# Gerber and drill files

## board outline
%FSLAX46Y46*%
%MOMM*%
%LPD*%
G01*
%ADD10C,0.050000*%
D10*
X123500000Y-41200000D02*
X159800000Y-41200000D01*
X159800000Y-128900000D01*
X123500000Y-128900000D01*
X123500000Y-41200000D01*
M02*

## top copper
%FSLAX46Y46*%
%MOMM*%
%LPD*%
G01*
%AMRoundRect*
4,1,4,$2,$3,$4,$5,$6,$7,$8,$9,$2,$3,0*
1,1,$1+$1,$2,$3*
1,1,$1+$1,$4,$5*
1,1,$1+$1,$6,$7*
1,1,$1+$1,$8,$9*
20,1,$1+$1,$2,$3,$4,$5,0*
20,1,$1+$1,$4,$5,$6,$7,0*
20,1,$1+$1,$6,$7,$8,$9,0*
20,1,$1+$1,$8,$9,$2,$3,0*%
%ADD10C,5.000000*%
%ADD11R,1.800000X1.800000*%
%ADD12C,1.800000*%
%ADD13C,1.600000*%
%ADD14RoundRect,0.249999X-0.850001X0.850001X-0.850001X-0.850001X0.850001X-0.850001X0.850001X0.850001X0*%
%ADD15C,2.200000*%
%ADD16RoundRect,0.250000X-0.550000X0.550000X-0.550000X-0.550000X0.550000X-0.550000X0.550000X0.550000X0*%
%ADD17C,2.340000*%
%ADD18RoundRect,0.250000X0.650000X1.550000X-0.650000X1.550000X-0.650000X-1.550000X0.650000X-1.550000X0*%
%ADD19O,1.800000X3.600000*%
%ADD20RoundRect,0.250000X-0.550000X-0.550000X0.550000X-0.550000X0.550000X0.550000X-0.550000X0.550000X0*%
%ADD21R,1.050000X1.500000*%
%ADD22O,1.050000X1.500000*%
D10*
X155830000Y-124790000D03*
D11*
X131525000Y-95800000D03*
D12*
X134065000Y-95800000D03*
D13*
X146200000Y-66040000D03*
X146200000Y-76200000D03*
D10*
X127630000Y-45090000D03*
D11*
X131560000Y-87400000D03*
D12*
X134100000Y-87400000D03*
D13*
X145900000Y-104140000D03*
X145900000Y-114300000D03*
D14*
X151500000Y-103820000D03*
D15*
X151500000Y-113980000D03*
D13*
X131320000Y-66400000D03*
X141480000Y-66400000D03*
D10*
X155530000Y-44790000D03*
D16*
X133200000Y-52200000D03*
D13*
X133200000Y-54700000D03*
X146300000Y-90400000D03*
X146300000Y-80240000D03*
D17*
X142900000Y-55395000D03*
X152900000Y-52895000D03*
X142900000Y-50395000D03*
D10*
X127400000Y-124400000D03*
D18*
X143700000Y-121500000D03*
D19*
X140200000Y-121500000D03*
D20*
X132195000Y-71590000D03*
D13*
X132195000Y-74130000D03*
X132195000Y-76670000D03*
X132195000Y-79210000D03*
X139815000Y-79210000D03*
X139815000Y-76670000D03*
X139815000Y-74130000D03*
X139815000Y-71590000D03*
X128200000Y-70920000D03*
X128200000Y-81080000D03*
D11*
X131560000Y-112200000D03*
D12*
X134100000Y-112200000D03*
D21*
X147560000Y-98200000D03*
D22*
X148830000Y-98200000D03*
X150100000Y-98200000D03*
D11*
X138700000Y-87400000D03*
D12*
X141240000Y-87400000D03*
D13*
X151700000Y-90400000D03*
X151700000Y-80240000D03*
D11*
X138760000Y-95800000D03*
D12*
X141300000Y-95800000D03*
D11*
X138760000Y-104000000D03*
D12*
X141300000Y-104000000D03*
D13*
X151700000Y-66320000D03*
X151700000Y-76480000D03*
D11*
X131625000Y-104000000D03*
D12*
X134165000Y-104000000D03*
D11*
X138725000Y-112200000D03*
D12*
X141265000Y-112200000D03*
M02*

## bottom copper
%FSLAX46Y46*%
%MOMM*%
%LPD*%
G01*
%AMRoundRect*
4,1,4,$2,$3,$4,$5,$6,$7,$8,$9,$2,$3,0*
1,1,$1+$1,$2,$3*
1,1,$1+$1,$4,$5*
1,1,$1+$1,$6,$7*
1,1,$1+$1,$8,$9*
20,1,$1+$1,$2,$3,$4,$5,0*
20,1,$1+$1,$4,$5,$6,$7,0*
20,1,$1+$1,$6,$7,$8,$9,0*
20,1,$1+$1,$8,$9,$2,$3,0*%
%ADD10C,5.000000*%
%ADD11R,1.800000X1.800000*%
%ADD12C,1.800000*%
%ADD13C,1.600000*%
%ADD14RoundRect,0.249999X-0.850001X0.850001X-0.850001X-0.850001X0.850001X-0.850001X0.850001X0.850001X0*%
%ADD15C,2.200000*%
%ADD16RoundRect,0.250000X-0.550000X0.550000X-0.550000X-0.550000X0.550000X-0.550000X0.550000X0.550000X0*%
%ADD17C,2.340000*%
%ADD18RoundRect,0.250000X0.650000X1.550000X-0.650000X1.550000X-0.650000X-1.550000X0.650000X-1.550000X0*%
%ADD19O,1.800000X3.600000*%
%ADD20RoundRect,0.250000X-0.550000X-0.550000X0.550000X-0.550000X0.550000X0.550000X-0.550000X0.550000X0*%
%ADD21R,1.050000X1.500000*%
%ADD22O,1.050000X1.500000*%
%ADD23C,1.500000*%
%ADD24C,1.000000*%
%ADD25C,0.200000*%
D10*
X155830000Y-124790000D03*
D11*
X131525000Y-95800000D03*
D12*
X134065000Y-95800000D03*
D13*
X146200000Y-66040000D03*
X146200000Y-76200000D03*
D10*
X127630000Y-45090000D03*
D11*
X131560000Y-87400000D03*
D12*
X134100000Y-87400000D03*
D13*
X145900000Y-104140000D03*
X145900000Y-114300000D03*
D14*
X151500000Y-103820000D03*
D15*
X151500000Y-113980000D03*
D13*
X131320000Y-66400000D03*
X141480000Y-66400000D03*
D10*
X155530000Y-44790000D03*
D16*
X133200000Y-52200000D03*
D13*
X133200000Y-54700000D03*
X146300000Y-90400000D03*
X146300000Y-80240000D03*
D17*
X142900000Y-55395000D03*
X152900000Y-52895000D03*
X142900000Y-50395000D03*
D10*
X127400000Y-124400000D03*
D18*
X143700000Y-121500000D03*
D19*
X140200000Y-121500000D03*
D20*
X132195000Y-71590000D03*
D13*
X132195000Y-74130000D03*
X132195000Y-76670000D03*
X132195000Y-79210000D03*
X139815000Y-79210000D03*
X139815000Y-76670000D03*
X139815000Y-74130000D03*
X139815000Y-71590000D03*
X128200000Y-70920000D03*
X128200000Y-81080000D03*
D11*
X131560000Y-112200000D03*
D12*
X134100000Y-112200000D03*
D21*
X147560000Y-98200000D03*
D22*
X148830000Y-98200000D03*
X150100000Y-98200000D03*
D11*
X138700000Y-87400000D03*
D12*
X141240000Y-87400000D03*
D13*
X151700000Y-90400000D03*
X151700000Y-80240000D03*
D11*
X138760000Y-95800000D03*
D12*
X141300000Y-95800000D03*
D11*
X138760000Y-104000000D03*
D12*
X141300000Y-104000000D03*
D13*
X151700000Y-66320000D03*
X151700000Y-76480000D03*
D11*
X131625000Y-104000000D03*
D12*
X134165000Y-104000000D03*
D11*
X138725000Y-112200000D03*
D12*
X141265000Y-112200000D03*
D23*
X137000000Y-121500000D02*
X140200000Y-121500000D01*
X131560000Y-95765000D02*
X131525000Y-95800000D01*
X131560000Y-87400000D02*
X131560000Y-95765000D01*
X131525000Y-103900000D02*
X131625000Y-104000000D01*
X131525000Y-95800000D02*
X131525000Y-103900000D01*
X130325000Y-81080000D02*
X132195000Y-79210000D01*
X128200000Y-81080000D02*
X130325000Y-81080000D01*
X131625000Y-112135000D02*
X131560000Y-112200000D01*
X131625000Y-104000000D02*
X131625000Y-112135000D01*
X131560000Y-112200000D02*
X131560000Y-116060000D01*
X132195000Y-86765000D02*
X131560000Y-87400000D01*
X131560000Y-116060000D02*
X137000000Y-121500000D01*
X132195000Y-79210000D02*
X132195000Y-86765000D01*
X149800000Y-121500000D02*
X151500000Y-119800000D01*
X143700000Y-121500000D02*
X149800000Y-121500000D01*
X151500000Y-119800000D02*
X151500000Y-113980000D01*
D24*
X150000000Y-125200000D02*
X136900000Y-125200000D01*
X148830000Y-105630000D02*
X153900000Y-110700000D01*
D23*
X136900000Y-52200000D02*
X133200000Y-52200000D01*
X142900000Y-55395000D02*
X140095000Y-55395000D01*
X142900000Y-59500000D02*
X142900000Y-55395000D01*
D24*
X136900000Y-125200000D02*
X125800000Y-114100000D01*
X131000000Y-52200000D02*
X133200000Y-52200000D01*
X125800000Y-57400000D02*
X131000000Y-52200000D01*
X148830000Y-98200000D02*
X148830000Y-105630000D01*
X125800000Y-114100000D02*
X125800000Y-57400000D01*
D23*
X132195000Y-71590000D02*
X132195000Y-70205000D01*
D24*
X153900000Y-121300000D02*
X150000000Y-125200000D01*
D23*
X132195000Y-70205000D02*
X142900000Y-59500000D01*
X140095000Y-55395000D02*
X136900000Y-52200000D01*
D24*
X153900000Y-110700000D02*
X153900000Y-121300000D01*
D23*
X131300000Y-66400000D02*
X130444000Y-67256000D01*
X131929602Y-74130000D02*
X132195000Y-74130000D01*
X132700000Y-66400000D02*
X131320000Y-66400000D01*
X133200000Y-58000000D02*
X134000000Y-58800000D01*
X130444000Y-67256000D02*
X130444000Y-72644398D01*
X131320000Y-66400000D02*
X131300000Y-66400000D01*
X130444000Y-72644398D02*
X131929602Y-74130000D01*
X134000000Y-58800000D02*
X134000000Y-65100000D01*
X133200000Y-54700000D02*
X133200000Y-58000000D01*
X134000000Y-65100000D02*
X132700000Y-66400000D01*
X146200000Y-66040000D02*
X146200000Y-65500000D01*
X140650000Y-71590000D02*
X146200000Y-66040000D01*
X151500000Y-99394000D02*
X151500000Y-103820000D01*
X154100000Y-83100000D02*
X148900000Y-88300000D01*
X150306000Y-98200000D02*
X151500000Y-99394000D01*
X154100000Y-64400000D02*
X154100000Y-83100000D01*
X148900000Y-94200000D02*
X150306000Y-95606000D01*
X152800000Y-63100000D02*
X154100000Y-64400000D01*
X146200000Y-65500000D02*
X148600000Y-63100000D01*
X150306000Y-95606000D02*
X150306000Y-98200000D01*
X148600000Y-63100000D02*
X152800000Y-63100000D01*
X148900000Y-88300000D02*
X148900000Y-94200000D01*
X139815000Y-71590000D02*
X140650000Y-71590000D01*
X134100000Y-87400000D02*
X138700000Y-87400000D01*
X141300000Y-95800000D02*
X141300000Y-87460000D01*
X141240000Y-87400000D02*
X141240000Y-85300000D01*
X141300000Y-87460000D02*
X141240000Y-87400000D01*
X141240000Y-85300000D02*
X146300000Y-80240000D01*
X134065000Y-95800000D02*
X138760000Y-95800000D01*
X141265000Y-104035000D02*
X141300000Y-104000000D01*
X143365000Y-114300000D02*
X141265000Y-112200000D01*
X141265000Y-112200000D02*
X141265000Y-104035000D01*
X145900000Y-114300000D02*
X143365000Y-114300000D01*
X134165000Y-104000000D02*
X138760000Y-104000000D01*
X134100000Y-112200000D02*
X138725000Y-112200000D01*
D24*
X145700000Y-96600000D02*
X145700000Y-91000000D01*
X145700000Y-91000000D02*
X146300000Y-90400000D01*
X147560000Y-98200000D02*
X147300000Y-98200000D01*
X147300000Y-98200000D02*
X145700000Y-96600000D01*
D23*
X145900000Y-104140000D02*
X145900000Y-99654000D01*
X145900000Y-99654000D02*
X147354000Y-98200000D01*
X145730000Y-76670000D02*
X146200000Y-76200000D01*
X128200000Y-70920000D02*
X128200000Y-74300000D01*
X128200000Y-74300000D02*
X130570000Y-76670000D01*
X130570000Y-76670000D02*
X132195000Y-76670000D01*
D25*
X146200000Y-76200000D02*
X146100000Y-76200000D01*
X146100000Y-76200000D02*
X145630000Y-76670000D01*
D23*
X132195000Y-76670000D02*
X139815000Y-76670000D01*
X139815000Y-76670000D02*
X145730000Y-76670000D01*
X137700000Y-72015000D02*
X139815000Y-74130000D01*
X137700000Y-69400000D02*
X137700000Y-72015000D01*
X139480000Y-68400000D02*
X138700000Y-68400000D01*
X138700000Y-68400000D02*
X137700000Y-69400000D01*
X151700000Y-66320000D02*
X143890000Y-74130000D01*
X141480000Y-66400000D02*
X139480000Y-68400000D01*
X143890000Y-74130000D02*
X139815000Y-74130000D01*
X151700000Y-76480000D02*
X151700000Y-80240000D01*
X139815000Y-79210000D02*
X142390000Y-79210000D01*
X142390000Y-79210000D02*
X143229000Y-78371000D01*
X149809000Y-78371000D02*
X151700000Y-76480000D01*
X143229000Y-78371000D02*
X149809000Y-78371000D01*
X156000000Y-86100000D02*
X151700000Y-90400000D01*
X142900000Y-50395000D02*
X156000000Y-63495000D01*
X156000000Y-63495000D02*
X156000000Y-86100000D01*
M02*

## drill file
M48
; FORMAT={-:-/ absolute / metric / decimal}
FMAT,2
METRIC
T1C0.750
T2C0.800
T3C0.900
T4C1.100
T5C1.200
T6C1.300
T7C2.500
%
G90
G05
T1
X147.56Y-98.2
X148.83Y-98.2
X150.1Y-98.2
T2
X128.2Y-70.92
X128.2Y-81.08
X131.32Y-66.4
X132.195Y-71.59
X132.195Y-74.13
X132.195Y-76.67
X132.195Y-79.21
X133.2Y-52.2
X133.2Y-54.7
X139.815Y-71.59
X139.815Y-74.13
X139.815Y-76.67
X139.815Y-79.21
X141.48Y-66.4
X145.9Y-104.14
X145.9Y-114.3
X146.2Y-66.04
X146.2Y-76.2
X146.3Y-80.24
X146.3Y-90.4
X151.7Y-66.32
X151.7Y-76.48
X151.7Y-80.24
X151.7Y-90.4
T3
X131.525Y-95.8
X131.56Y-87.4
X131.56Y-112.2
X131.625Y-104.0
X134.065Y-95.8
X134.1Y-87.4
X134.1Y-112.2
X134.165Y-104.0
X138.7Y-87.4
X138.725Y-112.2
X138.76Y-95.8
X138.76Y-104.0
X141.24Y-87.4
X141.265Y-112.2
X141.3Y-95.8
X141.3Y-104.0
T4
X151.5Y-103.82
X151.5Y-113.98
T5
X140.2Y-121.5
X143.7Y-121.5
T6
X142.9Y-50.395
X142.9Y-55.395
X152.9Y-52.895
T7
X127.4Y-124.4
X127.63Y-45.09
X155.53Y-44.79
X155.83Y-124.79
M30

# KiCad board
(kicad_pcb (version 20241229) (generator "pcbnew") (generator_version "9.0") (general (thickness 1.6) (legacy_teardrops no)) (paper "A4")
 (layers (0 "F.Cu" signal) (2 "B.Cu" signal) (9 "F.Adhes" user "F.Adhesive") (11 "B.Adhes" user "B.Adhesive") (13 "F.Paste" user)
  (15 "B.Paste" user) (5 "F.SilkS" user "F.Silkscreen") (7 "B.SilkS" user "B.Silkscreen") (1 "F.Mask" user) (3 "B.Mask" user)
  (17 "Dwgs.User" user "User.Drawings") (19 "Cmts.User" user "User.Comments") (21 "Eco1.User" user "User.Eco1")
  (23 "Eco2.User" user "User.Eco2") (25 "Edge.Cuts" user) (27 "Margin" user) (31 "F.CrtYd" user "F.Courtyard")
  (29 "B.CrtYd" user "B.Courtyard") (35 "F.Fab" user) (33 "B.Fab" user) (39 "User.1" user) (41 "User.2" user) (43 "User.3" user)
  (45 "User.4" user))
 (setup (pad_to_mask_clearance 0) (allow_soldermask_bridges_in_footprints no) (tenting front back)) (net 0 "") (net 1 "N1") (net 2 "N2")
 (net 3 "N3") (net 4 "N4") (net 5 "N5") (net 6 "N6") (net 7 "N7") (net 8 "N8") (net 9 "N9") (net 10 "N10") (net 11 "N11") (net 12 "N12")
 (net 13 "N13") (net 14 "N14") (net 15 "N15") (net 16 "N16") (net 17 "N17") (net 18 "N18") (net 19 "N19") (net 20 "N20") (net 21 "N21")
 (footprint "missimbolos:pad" (layer "F.Cu") (at 155.8 124.8)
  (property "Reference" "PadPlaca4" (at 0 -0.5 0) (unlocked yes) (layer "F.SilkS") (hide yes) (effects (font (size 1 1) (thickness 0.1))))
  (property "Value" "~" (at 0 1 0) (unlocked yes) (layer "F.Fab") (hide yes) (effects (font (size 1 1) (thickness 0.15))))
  (pad "1" thru_hole circle (at 0.03 -0.01) (size 5 5) (drill 2.5) (layers "*.Cu" "*.Mask") (remove_unused_layers no) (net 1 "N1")))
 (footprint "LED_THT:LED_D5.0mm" (layer "F.Cu") (at 131.525 95.8)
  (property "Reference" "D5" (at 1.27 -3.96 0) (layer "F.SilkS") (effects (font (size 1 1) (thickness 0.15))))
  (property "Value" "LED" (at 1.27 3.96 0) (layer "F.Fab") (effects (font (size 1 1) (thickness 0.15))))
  (pad "1" thru_hole rect (at 0 0) (size 1.8 1.8) (drill 0.9) (layers "*.Cu" "*.Mask") (remove_unused_layers no) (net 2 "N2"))
  (pad "2" thru_hole circle (at 2.54 0) (size 1.8 1.8) (drill 0.9) (layers "*.Cu" "*.Mask") (remove_unused_layers no) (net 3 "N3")))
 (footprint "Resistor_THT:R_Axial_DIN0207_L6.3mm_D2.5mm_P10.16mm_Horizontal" (layer "F.Cu") (at 146.2 66.04 -90)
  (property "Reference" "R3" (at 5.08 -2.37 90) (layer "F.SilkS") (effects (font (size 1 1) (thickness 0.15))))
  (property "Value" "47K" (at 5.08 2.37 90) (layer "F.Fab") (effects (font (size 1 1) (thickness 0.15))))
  (pad "1" thru_hole circle (at 0 0 270) (size 1.6 1.6) (drill 0.8) (layers "*.Cu" "*.Mask") (remove_unused_layers no) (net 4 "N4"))
  (pad "2" thru_hole circle (at 10.16 0 270) (size 1.6 1.6) (drill 0.8) (layers "*.Cu" "*.Mask") (remove_unused_layers no) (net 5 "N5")))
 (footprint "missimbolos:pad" (layer "F.Cu") (at 127.6 45.1)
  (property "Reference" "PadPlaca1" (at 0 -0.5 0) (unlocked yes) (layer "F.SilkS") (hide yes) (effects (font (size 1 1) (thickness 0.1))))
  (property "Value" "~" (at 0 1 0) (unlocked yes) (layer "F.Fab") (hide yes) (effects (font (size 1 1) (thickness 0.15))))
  (pad "1" thru_hole circle (at 0.03 -0.01) (size 5 5) (drill 2.5) (layers "*.Cu" "*.Mask") (remove_unused_layers no) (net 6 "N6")))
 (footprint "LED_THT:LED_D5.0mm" (layer "F.Cu") (at 131.56 87.4)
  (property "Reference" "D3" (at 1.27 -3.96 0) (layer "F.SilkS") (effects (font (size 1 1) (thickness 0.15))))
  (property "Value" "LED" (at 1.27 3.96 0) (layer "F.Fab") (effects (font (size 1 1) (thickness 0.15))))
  (pad "1" thru_hole rect (at 0 0) (size 1.8 1.8) (drill 0.9) (layers "*.Cu" "*.Mask") (remove_unused_layers no) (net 2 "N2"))
  (pad "2" thru_hole circle (at 2.54 0) (size 1.8 1.8) (drill 0.9) (layers "*.Cu" "*.Mask") (remove_unused_layers no) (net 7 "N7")))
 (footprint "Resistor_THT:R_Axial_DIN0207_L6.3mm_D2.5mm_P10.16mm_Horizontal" (layer "F.Cu") (at 145.9 104.14 -90)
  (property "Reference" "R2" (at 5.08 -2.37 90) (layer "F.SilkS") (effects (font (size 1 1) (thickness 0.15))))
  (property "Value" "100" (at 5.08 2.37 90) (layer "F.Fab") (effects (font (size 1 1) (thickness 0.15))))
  (pad "1" thru_hole circle (at 0 0 270) (size 1.6 1.6) (drill 0.8) (layers "*.Cu" "*.Mask") (remove_unused_layers no) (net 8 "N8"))
  (pad "2" thru_hole circle (at 10.16 0 270) (size 1.6 1.6) (drill 0.8) (layers "*.Cu" "*.Mask") (remove_unused_layers no) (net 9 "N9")))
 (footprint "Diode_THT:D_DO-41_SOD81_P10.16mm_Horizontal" (layer "F.Cu") (at 151.5 103.82 -90)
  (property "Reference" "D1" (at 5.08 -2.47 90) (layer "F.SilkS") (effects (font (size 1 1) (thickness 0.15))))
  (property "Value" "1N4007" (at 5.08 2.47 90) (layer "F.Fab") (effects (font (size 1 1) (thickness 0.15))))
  (pad "1" thru_hole roundrect (at 0 0 270) (size 2.2 2.2) (drill 1.1) (layers "*.Cu" "*.Mask") (remove_unused_layers no)
   (roundrect_rratio 0.113636) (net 4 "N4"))
  (pad "2" thru_hole circle (at 10.16 0 270) (size 2.2 2.2) (drill 1.1) (layers "*.Cu" "*.Mask") (remove_unused_layers no) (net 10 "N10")))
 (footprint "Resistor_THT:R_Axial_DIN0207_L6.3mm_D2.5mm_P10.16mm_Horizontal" (layer "F.Cu") (at 131.32 66.4)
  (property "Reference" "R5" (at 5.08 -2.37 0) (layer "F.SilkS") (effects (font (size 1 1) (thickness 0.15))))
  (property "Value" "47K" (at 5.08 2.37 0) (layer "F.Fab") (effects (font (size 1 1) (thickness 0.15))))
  (pad "1" thru_hole circle (at 0 0) (size 1.6 1.6) (drill 0.8) (layers "*.Cu" "*.Mask") (remove_unused_layers no) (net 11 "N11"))
  (pad "2" thru_hole circle (at 10.16 0) (size 1.6 1.6) (drill 0.8) (layers "*.Cu" "*.Mask") (remove_unused_layers no) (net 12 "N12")))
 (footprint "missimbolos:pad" (layer "F.Cu") (at 155.5 44.8)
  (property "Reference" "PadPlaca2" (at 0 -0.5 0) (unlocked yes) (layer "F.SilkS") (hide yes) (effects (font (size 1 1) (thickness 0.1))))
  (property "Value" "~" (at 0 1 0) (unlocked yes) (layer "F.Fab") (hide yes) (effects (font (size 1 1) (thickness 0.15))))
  (pad "1" thru_hole circle (at 0.03 -0.01) (size 5 5) (drill 2.5) (layers "*.Cu" "*.Mask") (remove_unused_layers no) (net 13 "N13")))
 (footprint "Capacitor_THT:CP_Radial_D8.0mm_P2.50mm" (layer "F.Cu") (at 133.2 52.2 -90)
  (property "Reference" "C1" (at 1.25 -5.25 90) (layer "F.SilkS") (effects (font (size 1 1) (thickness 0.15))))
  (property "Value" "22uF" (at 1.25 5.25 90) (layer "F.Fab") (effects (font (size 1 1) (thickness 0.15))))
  (pad "1" thru_hole roundrect (at 0 0 270) (size 1.6 1.6) (drill 0.8) (layers "*.Cu" "*.Mask") (remove_unused_layers no)
   (roundrect_rratio 0.15625) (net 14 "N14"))
  (pad "2" thru_hole circle (at 2.5 0 270) (size 1.6 1.6) (drill 0.8) (layers "*.Cu" "*.Mask") (remove_unused_layers no) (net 11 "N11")))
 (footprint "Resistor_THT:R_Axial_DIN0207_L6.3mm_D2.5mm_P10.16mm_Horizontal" (layer "F.Cu") (at 146.3 90.4 90)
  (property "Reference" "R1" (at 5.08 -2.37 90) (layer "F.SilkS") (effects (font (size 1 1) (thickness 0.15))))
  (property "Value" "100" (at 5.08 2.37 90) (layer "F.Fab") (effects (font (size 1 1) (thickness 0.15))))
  (pad "1" thru_hole circle (at 0 0 90) (size 1.6 1.6) (drill 0.8) (layers "*.Cu" "*.Mask") (remove_unused_layers no) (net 8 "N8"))
  (pad "2" thru_hole circle (at 10.16 0 90) (size 1.6 1.6) (drill 0.8) (layers "*.Cu" "*.Mask") (remove_unused_layers no) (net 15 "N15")))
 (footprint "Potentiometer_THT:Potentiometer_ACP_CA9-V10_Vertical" (layer "F.Cu") (at 142.9 55.395)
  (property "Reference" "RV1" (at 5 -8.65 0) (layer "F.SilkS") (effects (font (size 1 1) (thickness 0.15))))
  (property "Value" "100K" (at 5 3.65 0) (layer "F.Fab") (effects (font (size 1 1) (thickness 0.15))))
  (pad "1" thru_hole circle (at 0 0) (size 2.34 2.34) (drill 1.3) (layers "*.Cu" "*.Mask") (remove_unused_layers no) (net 14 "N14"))
  (pad "2" thru_hole circle (at 10 -2.5) (size 2.34 2.34) (drill 1.3) (layers "*.Cu" "*.Mask") (remove_unused_layers no) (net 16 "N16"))
  (pad "3" thru_hole circle (at 0 -5) (size 2.34 2.34) (drill 1.3) (layers "*.Cu" "*.Mask") (remove_unused_layers no) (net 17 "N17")))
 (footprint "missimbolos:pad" (layer "F.Cu") (at 127.37 124.41)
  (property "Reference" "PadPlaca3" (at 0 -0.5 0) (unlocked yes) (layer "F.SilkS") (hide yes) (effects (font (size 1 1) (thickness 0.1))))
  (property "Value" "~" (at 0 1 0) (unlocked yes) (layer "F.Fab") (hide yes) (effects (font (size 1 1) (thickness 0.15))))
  (pad "1" thru_hole circle (at 0.03 -0.01) (size 5 5) (drill 2.5) (layers "*.Cu" "*.Mask") (remove_unused_layers no) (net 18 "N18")))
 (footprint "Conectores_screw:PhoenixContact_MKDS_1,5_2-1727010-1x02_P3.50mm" (layer "F.Cu") (at 143.7 124.04 180)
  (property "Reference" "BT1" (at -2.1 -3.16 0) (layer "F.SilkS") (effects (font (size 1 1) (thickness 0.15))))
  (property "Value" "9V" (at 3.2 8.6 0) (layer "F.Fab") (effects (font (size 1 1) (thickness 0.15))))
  (pad "1" thru_hole roundrect (at 0 2.54 180) (size 1.8 3.6) (drill 1.2) (layers "*.Cu" "*.Mask") (remove_unused_layers no)
   (roundrect_rratio 0.138889) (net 10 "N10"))
  (pad "2" thru_hole oval (at 3.5 2.54 180) (size 1.8 3.6) (drill 1.2) (layers "*.Cu" "*.Mask") (remove_unused_layers no) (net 2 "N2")))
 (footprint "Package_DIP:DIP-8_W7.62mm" (layer "F.Cu") (at 132.195 71.59)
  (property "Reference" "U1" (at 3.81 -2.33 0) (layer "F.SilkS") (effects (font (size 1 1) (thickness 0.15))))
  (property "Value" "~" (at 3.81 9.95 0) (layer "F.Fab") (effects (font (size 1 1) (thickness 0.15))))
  (pad "1" thru_hole roundrect (at 0 0) (size 1.6 1.6) (drill 0.8) (layers "*.Cu" "*.Mask") (remove_unused_layers no)
   (roundrect_rratio 0.15625) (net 14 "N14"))
  (pad "2" thru_hole circle (at 0 2.54) (size 1.6 1.6) (drill 0.8) (layers "*.Cu" "*.Mask") (remove_unused_layers no) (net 11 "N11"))
  (pad "3" thru_hole circle (at 0 5.08) (size 1.6 1.6) (drill 0.8) (layers "*.Cu" "*.Mask") (remove_unused_layers no) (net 5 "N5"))
  (pad "4" thru_hole circle (at 0 7.62) (size 1.6 1.6) (drill 0.8) (layers "*.Cu" "*.Mask") (remove_unused_layers no) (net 2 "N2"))
  (pad "5" thru_hole circle (at 7.62 7.62) (size 1.6 1.6) (drill 0.8) (layers "*.Cu" "*.Mask") (remove_unused_layers no) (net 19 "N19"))
  (pad "6" thru_hole circle (at 7.62 5.08) (size 1.6 1.6) (drill 0.8) (layers "*.Cu" "*.Mask") (remove_unused_layers no) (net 5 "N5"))
  (pad "7" thru_hole circle (at 7.62 2.54) (size 1.6 1.6) (drill 0.8) (layers "*.Cu" "*.Mask") (remove_unused_layers no) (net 12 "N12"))
  (pad "8" thru_hole circle (at 7.62 0) (size 1.6 1.6) (drill 0.8) (layers "*.Cu" "*.Mask") (remove_unused_layers no) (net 4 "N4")))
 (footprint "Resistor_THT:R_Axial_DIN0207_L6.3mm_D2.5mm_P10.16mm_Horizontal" (layer "F.Cu") (at 128.2 70.92 -90)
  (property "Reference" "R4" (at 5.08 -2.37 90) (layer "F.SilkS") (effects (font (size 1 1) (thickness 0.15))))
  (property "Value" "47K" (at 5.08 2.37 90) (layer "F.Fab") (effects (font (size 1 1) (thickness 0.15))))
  (pad "1" thru_hole circle (at 0 0 270) (size 1.6 1.6) (drill 0.8) (layers "*.Cu" "*.Mask") (remove_unused_layers no) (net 5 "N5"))
  (pad "2" thru_hole circle (at 10.16 0 270) (size 1.6 1.6) (drill 0.8) (layers "*.Cu" "*.Mask") (remove_unused_layers no) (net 2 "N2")))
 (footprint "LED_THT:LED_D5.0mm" (layer "F.Cu") (at 131.56 112.2)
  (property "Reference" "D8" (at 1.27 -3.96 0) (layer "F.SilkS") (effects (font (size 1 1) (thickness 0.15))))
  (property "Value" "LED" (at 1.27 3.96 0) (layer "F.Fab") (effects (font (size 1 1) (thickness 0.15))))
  (pad "1" thru_hole rect (at 0 0) (size 1.8 1.8) (drill 0.9) (layers "*.Cu" "*.Mask") (remove_unused_layers no) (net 2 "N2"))
  (pad "2" thru_hole circle (at 2.54 0) (size 1.8 1.8) (drill 0.9) (layers "*.Cu" "*.Mask") (remove_unused_layers no) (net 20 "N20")))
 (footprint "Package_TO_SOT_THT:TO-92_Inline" (layer "F.Cu") (at 147.56 98.2)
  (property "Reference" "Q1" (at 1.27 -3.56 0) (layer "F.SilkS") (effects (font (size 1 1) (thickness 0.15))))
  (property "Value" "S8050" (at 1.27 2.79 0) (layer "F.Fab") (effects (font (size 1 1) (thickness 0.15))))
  (pad "1" thru_hole rect (at 0 0) (size 1.05 1.5) (drill 0.75) (layers "*.Cu" "*.Mask") (remove_unused_layers no) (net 8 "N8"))
  (pad "2" thru_hole oval (at 1.27 0) (size 1.05 1.5) (drill 0.75) (layers "*.Cu" "*.Mask") (remove_unused_layers no) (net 14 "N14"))
  (pad "3" thru_hole oval (at 2.54 0) (size 1.05 1.5) (drill 0.75) (layers "*.Cu" "*.Mask") (remove_unused_layers no) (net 4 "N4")))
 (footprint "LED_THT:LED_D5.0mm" (layer "F.Cu") (at 138.7 87.4)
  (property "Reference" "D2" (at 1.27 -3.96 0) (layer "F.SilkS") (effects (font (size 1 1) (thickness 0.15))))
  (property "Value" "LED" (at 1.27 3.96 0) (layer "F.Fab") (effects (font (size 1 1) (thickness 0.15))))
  (pad "1" thru_hole rect (at 0 0) (size 1.8 1.8) (drill 0.9) (layers "*.Cu" "*.Mask") (remove_unused_layers no) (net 7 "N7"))
  (pad "2" thru_hole circle (at 2.54 0) (size 1.8 1.8) (drill 0.9) (layers "*.Cu" "*.Mask") (remove_unused_layers no) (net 15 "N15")))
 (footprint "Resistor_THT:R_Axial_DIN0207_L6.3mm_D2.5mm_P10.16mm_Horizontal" (layer "F.Cu") (at 151.7 90.4 90)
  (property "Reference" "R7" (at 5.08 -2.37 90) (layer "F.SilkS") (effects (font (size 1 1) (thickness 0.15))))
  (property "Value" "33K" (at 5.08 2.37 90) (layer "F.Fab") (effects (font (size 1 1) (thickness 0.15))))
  (pad "1" thru_hole circle (at 0 0 90) (size 1.6 1.6) (drill 0.8) (layers "*.Cu" "*.Mask") (remove_unused_layers no) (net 17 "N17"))
  (pad "2" thru_hole circle (at 10.16 0 90) (size 1.6 1.6) (drill 0.8) (layers "*.Cu" "*.Mask") (remove_unused_layers no) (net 19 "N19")))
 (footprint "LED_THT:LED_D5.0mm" (layer "F.Cu") (at 138.76 95.8)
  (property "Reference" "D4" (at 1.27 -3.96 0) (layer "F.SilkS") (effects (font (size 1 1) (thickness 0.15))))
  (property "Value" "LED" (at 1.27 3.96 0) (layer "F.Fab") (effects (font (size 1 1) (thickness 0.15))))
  (pad "1" thru_hole rect (at 0 0) (size 1.8 1.8) (drill 0.9) (layers "*.Cu" "*.Mask") (remove_unused_layers no) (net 3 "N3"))
  (pad "2" thru_hole circle (at 2.54 0) (size 1.8 1.8) (drill 0.9) (layers "*.Cu" "*.Mask") (remove_unused_layers no) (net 15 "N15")))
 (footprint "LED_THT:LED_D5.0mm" (layer "F.Cu") (at 138.76 104)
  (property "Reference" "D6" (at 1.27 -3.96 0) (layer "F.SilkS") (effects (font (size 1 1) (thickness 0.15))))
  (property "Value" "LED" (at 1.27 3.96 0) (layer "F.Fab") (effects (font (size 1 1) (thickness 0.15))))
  (pad "1" thru_hole rect (at 0 0) (size 1.8 1.8) (drill 0.9) (layers "*.Cu" "*.Mask") (remove_unused_layers no) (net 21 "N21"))
  (pad "2" thru_hole circle (at 2.54 0) (size 1.8 1.8) (drill 0.9) (layers "*.Cu" "*.Mask") (remove_unused_layers no) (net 9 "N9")))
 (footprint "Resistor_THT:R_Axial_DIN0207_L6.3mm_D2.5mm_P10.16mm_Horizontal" (layer "F.Cu") (at 151.7 66.32 -90)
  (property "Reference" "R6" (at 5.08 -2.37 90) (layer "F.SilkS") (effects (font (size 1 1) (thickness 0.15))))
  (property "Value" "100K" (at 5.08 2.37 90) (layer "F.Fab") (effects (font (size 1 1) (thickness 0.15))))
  (pad "1" thru_hole circle (at 0 0 270) (size 1.6 1.6) (drill 0.8) (layers "*.Cu" "*.Mask") (remove_unused_layers no) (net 12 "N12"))
  (pad "2" thru_hole circle (at 10.16 0 270) (size 1.6 1.6) (drill 0.8) (layers "*.Cu" "*.Mask") (remove_unused_layers no) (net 19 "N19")))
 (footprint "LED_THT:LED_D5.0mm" (layer "F.Cu") (at 131.625 104)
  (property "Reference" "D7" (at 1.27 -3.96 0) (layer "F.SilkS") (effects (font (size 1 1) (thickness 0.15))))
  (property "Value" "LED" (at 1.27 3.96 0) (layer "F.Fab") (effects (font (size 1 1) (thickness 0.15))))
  (pad "1" thru_hole rect (at 0 0) (size 1.8 1.8) (drill 0.9) (layers "*.Cu" "*.Mask") (remove_unused_layers no) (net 2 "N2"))
  (pad "2" thru_hole circle (at 2.54 0) (size 1.8 1.8) (drill 0.9) (layers "*.Cu" "*.Mask") (remove_unused_layers no) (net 21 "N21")))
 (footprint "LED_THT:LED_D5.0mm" (layer "F.Cu") (at 138.725 112.2)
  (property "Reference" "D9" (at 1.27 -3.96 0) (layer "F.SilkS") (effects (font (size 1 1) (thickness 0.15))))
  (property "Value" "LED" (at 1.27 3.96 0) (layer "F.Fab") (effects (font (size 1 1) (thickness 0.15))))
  (pad "1" thru_hole rect (at 0 0) (size 1.8 1.8) (drill 0.9) (layers "*.Cu" "*.Mask") (remove_unused_layers no) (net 20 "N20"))
  (pad "2" thru_hole circle (at 2.54 0) (size 1.8 1.8) (drill 0.9) (layers "*.Cu" "*.Mask") (remove_unused_layers no) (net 9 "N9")))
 (gr_rect (start 123.5 41.2) (end 159.8 128.9) (stroke (width 0.05) (type default)) (fill no) (layer "Edge.Cuts"))
 (segment (start 137 121.5) (end 140.2 121.5) (width 1.5) (layer "B.Cu") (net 2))
 (segment (start 131.56 95.765) (end 131.525 95.8) (width 1.5) (layer "B.Cu") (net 2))
 (segment (start 131.56 87.4) (end 131.56 95.765) (width 1.5) (layer "B.Cu") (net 2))
 (segment (start 131.525 103.9) (end 131.625 104) (width 1.5) (layer "B.Cu") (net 2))
 (segment (start 131.525 95.8) (end 131.525 103.9) (width 1.5) (layer "B.Cu") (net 2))
 (segment (start 130.325 81.08) (end 132.195 79.21) (width 1.5) (layer "B.Cu") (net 2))
 (segment (start 128.2 81.08) (end 130.325 81.08) (width 1.5) (layer "B.Cu") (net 2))
 (segment (start 131.625 112.135) (end 131.56 112.2) (width 1.5) (layer "B.Cu") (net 2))
 (segment (start 131.625 104) (end 131.625 112.135) (width 1.5) (layer "B.Cu") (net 2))
 (segment (start 131.56 112.2) (end 131.56 116.06) (width 1.5) (layer "B.Cu") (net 2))
 (segment (start 132.195 86.765) (end 131.56 87.4) (width 1.5) (layer "B.Cu") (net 2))
 (segment (start 131.56 116.06) (end 137 121.5) (width 1.5) (layer "B.Cu") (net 2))
 (segment (start 132.195 79.21) (end 132.195 86.765) (width 1.5) (layer "B.Cu") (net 2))
 (segment (start 149.8 121.5) (end 151.5 119.8) (width 1.5) (layer "B.Cu") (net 10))
 (segment (start 143.7 121.5) (end 149.8 121.5) (width 1.5) (layer "B.Cu") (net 10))
 (segment (start 151.5 119.8) (end 151.5 113.98) (width 1.5) (layer "B.Cu") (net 10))
 (segment (start 150 125.2) (end 136.9 125.2) (width 1) (layer "B.Cu") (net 14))
 (segment (start 148.83 105.63) (end 153.9 110.7) (width 1) (layer "B.Cu") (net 14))
 (segment (start 136.9 52.2) (end 133.2 52.2) (width 1.5) (layer "B.Cu") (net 14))
 (segment (start 142.9 55.395) (end 140.095 55.395) (width 1.5) (layer "B.Cu") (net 14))
 (segment (start 142.9 59.5) (end 142.9 55.395) (width 1.5) (layer "B.Cu") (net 14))
 (segment (start 136.9 125.2) (end 125.8 114.1) (width 1) (layer "B.Cu") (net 14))
 (segment (start 131 52.2) (end 133.2 52.2) (width 1) (layer "B.Cu") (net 14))
 (segment (start 125.8 57.4) (end 131 52.2) (width 1) (layer "B.Cu") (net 14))
 (segment (start 148.83 98.2) (end 148.83 105.63) (width 1) (layer "B.Cu") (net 14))
 (segment (start 125.8 114.1) (end 125.8 57.4) (width 1) (layer "B.Cu") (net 14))
 (segment (start 132.195 71.59) (end 132.195 70.205) (width 1.5) (layer "B.Cu") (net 14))
 (segment (start 153.9 121.3) (end 150 125.2) (width 1) (layer "B.Cu") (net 14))
 (segment (start 132.195 70.205) (end 142.9 59.5) (width 1.5) (layer "B.Cu") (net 14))
 (segment (start 140.095 55.395) (end 136.9 52.2) (width 1.5) (layer "B.Cu") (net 14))
 (segment (start 153.9 110.7) (end 153.9 121.3) (width 1) (layer "B.Cu") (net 14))
 (segment (start 131.3 66.4) (end 130.444 67.256) (width 1.5) (layer "B.Cu") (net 11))
 (segment (start 131.929602 74.13) (end 132.195 74.13) (width 1.5) (layer "B.Cu") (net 11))
 (segment (start 132.7 66.4) (end 131.32 66.4) (width 1.5) (layer "B.Cu") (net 11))
 (segment (start 133.2 58) (end 134 58.8) (width 1.5) (layer "B.Cu") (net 11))
 (segment (start 130.444 67.256) (end 130.444 72.644398) (width 1.5) (layer "B.Cu") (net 11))
 (segment (start 131.32 66.4) (end 131.3 66.4) (width 1.5) (layer "B.Cu") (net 11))
 (segment (start 130.444 72.644398) (end 131.929602 74.13) (width 1.5) (layer "B.Cu") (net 11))
 (segment (start 134 58.8) (end 134 65.1) (width 1.5) (layer "B.Cu") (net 11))
 (segment (start 133.2 54.7) (end 133.2 58) (width 1.5) (layer "B.Cu") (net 11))
 (segment (start 134 65.1) (end 132.7 66.4) (width 1.5) (layer "B.Cu") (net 11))
 (segment (start 146.2 66.04) (end 146.2 65.5) (width 1.5) (layer "B.Cu") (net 4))
 (segment (start 140.65 71.59) (end 146.2 66.04) (width 1.5) (layer "B.Cu") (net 4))
 (segment (start 151.5 99.394) (end 151.5 103.82) (width 1.5) (layer "B.Cu") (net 4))
 (segment (start 154.1 83.1) (end 148.9 88.3) (width 1.5) (layer "B.Cu") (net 4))
 (segment (start 150.306 98.2) (end 151.5 99.394) (width 1.5) (layer "B.Cu") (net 4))
 (segment (start 154.1 64.4) (end 154.1 83.1) (width 1.5) (layer "B.Cu") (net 4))
 (segment (start 148.9 94.2) (end 150.306 95.606) (width 1.5) (layer "B.Cu") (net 4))
 (segment (start 152.8 63.1) (end 154.1 64.4) (width 1.5) (layer "B.Cu") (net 4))
 (segment (start 146.2 65.5) (end 148.6 63.1) (width 1.5) (layer "B.Cu") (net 4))
 (segment (start 150.306 95.606) (end 150.306 98.2) (width 1.5) (layer "B.Cu") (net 4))
 (segment (start 148.6 63.1) (end 152.8 63.1) (width 1.5) (layer "B.Cu") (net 4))
 (segment (start 148.9 88.3) (end 148.9 94.2) (width 1.5) (layer "B.Cu") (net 4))
 (segment (start 139.815 71.59) (end 140.65 71.59) (width 1.5) (layer "B.Cu") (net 4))
 (segment (start 134.1 87.4) (end 138.7 87.4) (width 1.5) (layer "B.Cu") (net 7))
 (segment (start 141.3 95.8) (end 141.3 87.46) (width 1.5) (layer "B.Cu") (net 15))
 (segment (start 141.24 87.4) (end 141.24 85.3) (width 1.5) (layer "B.Cu") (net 15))
 (segment (start 141.3 87.46) (end 141.24 87.4) (width 1.5) (layer "B.Cu") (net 15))
 (segment (start 141.24 85.3) (end 146.3 80.24) (width 1.5) (layer "B.Cu") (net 15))
 (segment (start 134.065 95.8) (end 138.76 95.8) (width 1.5) (layer "B.Cu") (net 3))
 (segment (start 141.265 104.035) (end 141.3 104) (width 1.5) (layer "B.Cu") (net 9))
 (segment (start 143.365 114.3) (end 141.265 112.2) (width 1.5) (layer "B.Cu") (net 9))
 (segment (start 141.265 112.2) (end 141.265 104.035) (width 1.5) (layer "B.Cu") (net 9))
 (segment (start 145.9 114.3) (end 143.365 114.3) (width 1.5) (layer "B.Cu") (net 9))
 (segment (start 134.165 104) (end 138.76 104) (width 1.5) (layer "B.Cu") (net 21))
 (segment (start 134.1 112.2) (end 138.725 112.2) (width 1.5) (layer "B.Cu") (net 20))
 (segment (start 145.7 96.6) (end 145.7 91) (width 1) (layer "B.Cu") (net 8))
 (segment (start 145.7 91) (end 146.3 90.4) (width 1) (layer "B.Cu") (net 8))
 (segment (start 147.56 98.2) (end 147.3 98.2) (width 1) (layer "B.Cu") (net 8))
 (segment (start 147.3 98.2) (end 145.7 96.6) (width 1) (layer "B.Cu") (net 8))
 (segment (start 145.9 104.14) (end 145.9 99.654) (width 1.5) (layer "B.Cu") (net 8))
 (segment (start 145.9 99.654) (end 147.354 98.2) (width 1.5) (layer "B.Cu") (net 8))
 (segment (start 145.73 76.67) (end 146.2 76.2) (width 1.5) (layer "B.Cu") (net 5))
 (segment (start 128.2 70.92) (end 128.2 74.3) (width 1.5) (layer "B.Cu") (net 5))
 (segment (start 128.2 74.3) (end 130.57 76.67) (width 1.5) (layer "B.Cu") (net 5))
 (segment (start 130.57 76.67) (end 132.195 76.67) (width 1.5) (layer "B.Cu") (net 5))
 (segment (start 146.2 76.2) (end 146.1 76.2) (width 0.2) (layer "B.Cu") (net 5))
 (segment (start 146.1 76.2) (end 145.63 76.67) (width 0.2) (layer "B.Cu") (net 5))
 (segment (start 132.195 76.67) (end 139.815 76.67) (width 1.5) (layer "B.Cu") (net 5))
 (segment (start 139.815 76.67) (end 145.73 76.67) (width 1.5) (layer "B.Cu") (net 5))
 (segment (start 137.7 72.015) (end 139.815 74.13) (width 1.5) (layer "B.Cu") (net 12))
 (segment (start 137.7 69.4) (end 137.7 72.015) (width 1.5) (layer "B.Cu") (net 12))
 (segment (start 139.48 68.4) (end 138.7 68.4) (width 1.5) (layer "B.Cu") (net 12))
 (segment (start 138.7 68.4) (end 137.7 69.4) (width 1.5) (layer "B.Cu") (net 12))
 (segment (start 151.7 66.32) (end 143.89 74.13) (width 1.5) (layer "B.Cu") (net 12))
 (segment (start 141.48 66.4) (end 139.48 68.4) (width 1.5) (layer "B.Cu") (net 12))
 (segment (start 143.89 74.13) (end 139.815 74.13) (width 1.5) (layer "B.Cu") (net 12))
 (segment (start 151.7 76.48) (end 151.7 80.24) (width 1.5) (layer "B.Cu") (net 19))
 (segment (start 139.815 79.21) (end 142.39 79.21) (width 1.5) (layer "B.Cu") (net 19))
 (segment (start 142.39 79.21) (end 143.229 78.371) (width 1.5) (layer "B.Cu") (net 19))
 (segment (start 149.809 78.371) (end 151.7 76.48) (width 1.5) (layer "B.Cu") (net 19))
 (segment (start 143.229 78.371) (end 149.809 78.371) (width 1.5) (layer "B.Cu") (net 19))
 (segment (start 156 86.1) (end 151.7 90.4) (width 1.5) (layer "B.Cu") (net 17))
 (segment (start 142.9 50.395) (end 156 63.495) (width 1.5) (layer "B.Cu") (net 17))
 (segment (start 156 63.495) (end 156 86.1) (width 1.5) (layer "B.Cu") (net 17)))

